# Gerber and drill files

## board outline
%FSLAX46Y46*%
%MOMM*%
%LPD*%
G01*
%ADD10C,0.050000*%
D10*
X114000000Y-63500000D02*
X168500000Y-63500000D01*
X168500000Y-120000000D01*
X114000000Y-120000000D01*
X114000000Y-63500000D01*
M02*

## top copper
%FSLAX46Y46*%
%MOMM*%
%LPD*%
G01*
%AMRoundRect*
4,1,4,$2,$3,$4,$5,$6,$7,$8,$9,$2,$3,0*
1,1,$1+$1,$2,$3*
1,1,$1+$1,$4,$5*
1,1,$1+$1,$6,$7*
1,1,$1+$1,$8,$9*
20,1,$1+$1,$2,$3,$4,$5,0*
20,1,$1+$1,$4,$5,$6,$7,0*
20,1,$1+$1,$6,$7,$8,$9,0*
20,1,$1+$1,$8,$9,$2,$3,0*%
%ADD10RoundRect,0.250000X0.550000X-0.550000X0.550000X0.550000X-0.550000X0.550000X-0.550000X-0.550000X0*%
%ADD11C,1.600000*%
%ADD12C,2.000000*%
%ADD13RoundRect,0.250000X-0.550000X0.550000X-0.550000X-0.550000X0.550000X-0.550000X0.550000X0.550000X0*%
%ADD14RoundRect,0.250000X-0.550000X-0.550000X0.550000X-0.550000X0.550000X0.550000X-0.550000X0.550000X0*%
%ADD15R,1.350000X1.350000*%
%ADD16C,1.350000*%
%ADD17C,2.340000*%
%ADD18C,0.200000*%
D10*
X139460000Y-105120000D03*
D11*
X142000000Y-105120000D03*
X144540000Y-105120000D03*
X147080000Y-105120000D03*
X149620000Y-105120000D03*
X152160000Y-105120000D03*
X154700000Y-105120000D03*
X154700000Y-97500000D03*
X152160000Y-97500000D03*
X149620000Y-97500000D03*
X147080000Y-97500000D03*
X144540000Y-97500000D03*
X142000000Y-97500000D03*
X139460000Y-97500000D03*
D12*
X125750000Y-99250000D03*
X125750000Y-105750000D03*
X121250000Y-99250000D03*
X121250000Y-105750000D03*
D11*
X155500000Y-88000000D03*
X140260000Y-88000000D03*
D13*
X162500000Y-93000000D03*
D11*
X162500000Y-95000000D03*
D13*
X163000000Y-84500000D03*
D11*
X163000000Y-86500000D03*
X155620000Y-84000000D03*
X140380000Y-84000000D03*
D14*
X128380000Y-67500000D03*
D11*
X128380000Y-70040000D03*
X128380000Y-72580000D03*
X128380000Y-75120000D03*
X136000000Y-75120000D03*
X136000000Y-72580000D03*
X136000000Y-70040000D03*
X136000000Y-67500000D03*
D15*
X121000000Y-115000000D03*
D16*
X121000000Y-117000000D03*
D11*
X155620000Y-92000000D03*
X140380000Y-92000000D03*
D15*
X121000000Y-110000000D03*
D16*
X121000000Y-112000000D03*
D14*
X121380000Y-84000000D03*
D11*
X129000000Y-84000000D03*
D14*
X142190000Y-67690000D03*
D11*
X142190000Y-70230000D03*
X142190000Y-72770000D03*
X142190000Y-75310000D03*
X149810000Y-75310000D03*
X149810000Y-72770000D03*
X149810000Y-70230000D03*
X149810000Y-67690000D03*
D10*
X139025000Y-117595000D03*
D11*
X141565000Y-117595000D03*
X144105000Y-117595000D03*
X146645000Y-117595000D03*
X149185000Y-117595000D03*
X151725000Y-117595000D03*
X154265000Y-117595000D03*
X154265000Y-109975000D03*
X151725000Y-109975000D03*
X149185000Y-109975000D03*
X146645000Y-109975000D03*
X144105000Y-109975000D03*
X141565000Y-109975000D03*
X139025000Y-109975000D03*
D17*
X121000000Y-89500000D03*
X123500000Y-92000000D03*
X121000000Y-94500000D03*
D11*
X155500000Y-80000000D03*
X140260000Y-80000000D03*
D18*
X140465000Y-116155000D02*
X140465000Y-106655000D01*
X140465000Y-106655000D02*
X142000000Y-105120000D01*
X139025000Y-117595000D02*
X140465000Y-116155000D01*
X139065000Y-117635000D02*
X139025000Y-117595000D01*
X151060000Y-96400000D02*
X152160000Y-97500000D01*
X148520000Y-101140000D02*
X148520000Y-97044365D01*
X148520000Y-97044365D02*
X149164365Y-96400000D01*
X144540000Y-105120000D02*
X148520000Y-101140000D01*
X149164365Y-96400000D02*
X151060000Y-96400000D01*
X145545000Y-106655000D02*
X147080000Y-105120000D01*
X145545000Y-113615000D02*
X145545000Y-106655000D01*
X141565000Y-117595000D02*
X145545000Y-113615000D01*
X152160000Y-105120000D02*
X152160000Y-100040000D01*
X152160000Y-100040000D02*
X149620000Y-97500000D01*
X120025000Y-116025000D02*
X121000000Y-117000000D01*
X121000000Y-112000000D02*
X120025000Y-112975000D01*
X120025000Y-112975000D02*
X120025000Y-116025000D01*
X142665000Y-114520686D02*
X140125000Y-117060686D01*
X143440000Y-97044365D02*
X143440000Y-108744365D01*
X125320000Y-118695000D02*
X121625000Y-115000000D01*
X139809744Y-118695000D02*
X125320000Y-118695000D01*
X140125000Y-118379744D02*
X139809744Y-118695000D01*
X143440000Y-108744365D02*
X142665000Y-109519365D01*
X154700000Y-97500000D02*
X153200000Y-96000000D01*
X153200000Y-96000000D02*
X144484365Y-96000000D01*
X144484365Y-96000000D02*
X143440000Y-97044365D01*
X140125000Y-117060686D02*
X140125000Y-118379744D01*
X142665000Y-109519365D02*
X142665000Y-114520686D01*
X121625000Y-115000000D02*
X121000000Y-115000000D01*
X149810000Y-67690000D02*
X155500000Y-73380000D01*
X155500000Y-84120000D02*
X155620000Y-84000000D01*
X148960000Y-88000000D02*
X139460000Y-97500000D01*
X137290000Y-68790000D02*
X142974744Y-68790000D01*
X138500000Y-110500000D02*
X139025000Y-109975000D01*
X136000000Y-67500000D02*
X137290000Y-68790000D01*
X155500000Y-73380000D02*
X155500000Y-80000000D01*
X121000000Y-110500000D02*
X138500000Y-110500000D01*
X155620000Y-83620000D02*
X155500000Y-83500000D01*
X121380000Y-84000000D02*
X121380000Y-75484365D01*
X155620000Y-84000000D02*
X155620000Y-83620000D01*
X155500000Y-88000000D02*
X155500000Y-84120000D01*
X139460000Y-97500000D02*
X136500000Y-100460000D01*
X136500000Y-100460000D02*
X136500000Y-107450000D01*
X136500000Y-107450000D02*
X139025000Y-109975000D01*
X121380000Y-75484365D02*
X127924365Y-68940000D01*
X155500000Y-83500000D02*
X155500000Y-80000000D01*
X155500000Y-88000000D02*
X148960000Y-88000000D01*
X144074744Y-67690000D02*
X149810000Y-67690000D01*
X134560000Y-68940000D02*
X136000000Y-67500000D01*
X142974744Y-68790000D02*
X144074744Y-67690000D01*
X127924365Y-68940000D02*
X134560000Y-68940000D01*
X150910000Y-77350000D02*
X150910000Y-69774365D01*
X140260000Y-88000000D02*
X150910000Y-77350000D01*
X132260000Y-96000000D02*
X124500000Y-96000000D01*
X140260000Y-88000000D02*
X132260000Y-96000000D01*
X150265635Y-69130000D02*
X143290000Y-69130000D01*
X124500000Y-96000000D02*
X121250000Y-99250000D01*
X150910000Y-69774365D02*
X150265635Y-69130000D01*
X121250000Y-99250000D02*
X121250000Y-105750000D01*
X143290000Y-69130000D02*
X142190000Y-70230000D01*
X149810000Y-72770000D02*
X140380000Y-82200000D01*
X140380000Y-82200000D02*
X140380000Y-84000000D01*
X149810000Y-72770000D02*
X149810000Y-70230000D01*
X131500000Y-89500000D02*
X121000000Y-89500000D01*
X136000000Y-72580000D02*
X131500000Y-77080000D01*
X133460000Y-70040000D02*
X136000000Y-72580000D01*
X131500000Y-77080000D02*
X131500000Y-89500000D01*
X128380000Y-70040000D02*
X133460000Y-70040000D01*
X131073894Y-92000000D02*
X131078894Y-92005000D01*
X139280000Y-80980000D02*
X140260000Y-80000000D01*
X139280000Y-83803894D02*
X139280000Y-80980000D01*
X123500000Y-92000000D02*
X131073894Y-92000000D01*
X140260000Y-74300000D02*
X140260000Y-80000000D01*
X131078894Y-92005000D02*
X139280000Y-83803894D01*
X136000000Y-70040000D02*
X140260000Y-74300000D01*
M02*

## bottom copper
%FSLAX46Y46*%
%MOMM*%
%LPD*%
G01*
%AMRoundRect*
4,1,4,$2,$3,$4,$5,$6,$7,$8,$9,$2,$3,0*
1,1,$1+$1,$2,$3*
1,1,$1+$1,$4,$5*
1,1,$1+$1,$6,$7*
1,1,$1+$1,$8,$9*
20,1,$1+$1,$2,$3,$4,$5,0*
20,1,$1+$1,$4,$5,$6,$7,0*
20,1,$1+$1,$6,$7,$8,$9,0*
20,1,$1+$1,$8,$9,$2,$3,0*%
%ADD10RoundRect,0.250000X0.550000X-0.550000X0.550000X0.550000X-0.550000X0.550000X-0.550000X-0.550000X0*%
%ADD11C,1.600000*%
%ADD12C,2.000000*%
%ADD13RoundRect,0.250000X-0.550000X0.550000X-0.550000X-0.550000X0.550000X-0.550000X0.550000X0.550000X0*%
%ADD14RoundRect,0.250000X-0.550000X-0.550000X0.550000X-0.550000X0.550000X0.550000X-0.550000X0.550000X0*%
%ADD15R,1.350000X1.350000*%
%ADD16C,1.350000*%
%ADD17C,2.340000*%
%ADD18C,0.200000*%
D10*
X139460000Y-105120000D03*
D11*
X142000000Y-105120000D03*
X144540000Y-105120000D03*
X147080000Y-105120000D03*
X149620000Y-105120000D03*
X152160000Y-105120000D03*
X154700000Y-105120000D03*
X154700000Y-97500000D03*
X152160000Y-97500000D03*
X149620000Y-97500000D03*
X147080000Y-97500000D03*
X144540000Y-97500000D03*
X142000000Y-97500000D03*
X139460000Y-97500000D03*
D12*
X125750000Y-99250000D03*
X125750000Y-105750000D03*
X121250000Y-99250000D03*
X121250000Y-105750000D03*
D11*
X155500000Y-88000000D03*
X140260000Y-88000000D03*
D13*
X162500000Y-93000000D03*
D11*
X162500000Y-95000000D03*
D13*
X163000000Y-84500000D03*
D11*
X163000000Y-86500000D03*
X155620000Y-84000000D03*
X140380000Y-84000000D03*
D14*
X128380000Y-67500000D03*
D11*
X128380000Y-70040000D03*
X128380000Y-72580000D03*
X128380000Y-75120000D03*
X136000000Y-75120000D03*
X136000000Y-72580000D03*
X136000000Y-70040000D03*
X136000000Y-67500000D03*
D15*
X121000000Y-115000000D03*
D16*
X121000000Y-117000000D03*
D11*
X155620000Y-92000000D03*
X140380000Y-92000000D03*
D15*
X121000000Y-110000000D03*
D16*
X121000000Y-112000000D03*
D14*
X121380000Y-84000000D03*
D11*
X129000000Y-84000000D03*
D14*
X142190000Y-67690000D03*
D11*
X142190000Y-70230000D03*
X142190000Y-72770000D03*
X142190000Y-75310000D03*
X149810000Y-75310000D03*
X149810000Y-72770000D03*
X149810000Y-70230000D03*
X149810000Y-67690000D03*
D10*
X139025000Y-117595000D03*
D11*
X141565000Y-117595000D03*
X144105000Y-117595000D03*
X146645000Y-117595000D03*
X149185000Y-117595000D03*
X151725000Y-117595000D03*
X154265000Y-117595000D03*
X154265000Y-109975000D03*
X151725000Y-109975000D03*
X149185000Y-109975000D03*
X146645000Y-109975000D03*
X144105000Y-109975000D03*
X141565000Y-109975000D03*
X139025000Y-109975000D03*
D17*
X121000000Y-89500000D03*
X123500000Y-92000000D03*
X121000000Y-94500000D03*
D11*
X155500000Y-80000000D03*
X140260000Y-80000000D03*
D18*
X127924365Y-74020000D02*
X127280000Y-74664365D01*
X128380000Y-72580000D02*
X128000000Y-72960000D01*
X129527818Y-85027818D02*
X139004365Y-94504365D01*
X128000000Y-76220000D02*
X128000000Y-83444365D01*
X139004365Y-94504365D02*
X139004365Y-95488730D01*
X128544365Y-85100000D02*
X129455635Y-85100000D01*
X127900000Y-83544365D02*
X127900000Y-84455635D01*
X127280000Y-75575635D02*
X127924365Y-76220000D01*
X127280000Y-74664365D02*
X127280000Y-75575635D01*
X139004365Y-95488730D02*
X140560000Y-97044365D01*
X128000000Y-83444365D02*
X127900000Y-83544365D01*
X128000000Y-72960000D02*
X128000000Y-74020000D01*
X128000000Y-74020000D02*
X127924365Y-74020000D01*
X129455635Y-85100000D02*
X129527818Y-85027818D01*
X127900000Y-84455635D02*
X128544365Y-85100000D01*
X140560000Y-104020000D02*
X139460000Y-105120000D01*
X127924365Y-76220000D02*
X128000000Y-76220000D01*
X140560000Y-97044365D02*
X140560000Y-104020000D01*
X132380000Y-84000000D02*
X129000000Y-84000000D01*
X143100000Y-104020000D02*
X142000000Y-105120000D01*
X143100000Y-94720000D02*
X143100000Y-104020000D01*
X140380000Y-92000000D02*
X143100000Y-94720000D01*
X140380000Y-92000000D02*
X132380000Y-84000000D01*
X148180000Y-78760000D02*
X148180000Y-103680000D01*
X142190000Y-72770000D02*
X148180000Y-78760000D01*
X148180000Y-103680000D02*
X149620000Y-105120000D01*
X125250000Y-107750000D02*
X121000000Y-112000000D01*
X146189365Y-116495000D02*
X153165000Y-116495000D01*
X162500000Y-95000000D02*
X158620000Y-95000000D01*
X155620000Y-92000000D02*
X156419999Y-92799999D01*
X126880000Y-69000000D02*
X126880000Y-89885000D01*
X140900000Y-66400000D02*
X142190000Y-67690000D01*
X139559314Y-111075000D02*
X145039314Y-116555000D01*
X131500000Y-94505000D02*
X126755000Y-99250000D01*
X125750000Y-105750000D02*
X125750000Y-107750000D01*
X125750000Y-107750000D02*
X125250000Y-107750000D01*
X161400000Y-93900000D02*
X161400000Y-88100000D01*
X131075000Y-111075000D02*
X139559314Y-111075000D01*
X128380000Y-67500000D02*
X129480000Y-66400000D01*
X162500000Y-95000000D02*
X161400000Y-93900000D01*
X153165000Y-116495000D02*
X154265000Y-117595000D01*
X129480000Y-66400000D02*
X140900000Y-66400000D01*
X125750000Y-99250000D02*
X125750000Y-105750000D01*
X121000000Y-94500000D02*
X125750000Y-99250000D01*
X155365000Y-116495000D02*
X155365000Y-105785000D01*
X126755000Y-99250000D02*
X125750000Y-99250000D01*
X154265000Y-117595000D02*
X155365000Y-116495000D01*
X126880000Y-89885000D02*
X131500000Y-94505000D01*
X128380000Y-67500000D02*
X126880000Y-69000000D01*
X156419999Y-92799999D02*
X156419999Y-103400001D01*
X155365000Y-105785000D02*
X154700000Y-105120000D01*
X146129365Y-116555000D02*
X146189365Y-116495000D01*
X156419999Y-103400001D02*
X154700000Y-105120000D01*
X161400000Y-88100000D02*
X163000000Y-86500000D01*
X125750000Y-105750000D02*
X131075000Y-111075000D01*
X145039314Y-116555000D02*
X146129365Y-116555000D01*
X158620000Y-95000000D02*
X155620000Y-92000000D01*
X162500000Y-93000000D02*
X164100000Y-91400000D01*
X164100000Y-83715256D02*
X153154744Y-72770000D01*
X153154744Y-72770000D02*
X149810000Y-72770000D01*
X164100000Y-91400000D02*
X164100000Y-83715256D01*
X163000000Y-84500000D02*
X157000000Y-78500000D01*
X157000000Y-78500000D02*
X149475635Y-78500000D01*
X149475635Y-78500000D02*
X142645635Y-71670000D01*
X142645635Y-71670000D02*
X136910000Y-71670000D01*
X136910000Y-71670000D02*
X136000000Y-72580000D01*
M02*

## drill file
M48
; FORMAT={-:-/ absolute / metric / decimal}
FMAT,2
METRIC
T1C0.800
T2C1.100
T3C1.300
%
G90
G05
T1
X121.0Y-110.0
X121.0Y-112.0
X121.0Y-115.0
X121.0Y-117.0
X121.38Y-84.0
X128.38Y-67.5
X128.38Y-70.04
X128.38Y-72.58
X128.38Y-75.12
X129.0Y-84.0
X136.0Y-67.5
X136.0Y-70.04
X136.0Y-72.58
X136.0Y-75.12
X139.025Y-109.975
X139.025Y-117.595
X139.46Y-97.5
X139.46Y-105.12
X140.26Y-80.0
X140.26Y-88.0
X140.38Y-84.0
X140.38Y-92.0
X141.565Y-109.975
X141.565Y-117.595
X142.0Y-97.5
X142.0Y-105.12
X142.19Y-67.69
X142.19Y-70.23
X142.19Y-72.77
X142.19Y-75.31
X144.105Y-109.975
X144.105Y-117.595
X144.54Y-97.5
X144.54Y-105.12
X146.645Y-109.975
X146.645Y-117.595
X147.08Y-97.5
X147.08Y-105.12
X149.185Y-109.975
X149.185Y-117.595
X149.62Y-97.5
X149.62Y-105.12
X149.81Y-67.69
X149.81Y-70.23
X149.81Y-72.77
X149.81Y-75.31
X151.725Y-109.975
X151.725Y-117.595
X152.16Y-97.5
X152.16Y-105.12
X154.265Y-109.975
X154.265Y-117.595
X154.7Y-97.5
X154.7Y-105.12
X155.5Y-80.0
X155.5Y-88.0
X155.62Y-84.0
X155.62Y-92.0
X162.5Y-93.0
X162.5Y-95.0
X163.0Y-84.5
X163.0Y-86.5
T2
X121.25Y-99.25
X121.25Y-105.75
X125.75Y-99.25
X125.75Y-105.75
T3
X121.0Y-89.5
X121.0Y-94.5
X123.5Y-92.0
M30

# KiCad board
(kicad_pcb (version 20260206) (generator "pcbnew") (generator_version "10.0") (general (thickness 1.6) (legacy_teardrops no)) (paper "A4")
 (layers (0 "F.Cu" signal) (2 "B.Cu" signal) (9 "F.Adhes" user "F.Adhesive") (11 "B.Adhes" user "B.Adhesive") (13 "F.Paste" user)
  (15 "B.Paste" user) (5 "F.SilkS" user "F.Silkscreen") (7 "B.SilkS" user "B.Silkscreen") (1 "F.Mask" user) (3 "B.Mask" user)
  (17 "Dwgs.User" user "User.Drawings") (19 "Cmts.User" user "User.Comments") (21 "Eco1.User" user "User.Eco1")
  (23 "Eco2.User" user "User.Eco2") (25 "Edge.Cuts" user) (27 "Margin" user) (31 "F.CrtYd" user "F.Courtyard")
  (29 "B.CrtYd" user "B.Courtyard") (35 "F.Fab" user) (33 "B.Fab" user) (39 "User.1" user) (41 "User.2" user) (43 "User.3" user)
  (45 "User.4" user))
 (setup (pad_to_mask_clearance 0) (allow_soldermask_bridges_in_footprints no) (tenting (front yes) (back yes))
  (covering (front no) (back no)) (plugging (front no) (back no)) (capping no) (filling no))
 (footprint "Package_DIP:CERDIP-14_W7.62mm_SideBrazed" (layer "F.Cu") (at 139.46 105.12 90)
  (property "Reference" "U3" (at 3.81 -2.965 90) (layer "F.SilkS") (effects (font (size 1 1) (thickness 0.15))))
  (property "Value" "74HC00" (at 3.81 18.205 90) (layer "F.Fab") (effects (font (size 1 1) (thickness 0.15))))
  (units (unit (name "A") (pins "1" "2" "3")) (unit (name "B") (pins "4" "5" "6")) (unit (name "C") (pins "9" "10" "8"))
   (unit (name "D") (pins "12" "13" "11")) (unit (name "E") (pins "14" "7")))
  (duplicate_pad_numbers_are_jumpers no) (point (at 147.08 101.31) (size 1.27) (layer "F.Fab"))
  (pad "1" thru_hole roundrect (at 0 0 90) (size 1.6 1.6) (drill 0.8) (layers "*.Cu" "*.Mask") (remove_unused_layers no)
   (roundrect_rratio 0.15625) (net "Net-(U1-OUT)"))
  (pad "2" thru_hole circle (at 0 2.54 90) (size 1.6 1.6) (drill 0.8) (layers "*.Cu" "*.Mask") (remove_unused_layers no)
   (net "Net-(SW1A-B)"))
  (pad "3" thru_hole circle (at 0 5.08 90) (size 1.6 1.6) (drill 0.8) (layers "*.Cu" "*.Mask") (remove_unused_layers no)
   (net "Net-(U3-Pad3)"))
  (pad "4" thru_hole circle (at 0 7.62 90) (size 1.6 1.6) (drill 0.8) (layers "*.Cu" "*.Mask") (remove_unused_layers no)
   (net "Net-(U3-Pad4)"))
  (pad "5" thru_hole circle (at 0 10.16 90) (size 1.6 1.6) (drill 0.8) (layers "*.Cu" "*.Mask") (remove_unused_layers no)
   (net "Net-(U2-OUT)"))
  (pad "6" thru_hole circle (at 0 12.7 90) (size 1.6 1.6) (drill 0.8) (layers "*.Cu" "*.Mask") (remove_unused_layers no)
   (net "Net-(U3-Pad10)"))
  (pad "7" thru_hole circle (at 0 15.24 90) (size 1.6 1.6) (drill 0.8) (layers "*.Cu" "*.Mask") (remove_unused_layers no) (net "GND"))
  (pad "8" thru_hole circle (at 7.62 15.24 90) (size 1.6 1.6) (drill 0.8) (layers "*.Cu" "*.Mask") (remove_unused_layers no)
   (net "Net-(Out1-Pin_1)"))
  (pad "9" thru_hole circle (at 7.62 12.7 90) (size 1.6 1.6) (drill 0.8) (layers "*.Cu" "*.Mask") (remove_unused_layers no)
   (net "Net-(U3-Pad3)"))
  (pad "10" thru_hole circle (at 7.62 10.16 90) (size 1.6 1.6) (drill 0.8) (layers "*.Cu" "*.Mask") (remove_unused_layers no)
   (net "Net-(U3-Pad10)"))
  (pad "11" thru_hole circle (at 7.62 7.62 90) (size 1.6 1.6) (drill 0.8) (layers "*.Cu" "*.Mask") (remove_unused_layers no))
  (pad "12" thru_hole circle (at 7.62 5.08 90) (size 1.6 1.6) (drill 0.8) (layers "*.Cu" "*.Mask") (remove_unused_layers no))
  (pad "13" thru_hole circle (at 7.62 2.54 90) (size 1.6 1.6) (drill 0.8) (layers "*.Cu" "*.Mask") (remove_unused_layers no))
  (pad "14" thru_hole circle (at 7.62 0 90) (size 1.6 1.6) (drill 0.8) (layers "*.Cu" "*.Mask") (remove_unused_layers no) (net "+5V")))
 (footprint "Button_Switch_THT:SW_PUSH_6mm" (layer "F.Cu") (at 125.75 99.25 -90)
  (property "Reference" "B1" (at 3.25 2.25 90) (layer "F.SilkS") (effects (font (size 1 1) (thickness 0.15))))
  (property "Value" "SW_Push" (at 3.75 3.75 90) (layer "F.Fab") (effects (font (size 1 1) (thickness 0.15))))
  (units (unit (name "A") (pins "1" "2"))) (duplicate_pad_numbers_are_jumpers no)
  (pad "1" thru_hole circle (at 0 0) (size 2 2) (drill 1.1) (layers "*.Cu" "*.Mask") (remove_unused_layers no) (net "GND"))
  (pad "1" thru_hole circle (at 6.5 0) (size 2 2) (drill 1.1) (layers "*.Cu" "*.Mask") (remove_unused_layers no) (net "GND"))
  (pad "2" thru_hole circle (at 0 4.5) (size 2 2) (drill 1.1) (layers "*.Cu" "*.Mask") (remove_unused_layers no) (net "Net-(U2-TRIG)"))
  (pad "2" thru_hole circle (at 6.5 4.5) (size 2 2) (drill 1.1) (layers "*.Cu" "*.Mask") (remove_unused_layers no) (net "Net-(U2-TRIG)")))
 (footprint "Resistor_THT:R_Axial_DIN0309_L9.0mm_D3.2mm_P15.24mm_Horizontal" (layer "F.Cu") (at 155.5 88 180)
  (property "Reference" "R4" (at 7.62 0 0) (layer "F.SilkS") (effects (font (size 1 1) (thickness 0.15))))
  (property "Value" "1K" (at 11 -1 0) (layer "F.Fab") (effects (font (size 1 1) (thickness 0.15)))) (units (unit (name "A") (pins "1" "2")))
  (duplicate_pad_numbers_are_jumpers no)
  (pad "1" thru_hole circle (at 0 0 180) (size 1.6 1.6) (drill 0.8) (layers "*.Cu" "*.Mask") (remove_unused_layers no) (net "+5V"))
  (pad "2" thru_hole circle (at 15.24 0 180) (size 1.6 1.6) (drill 0.8) (layers "*.Cu" "*.Mask") (remove_unused_layers no)
   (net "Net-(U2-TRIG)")))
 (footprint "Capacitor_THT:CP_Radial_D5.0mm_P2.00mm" (layer "F.Cu") (at 162.5 93 -90)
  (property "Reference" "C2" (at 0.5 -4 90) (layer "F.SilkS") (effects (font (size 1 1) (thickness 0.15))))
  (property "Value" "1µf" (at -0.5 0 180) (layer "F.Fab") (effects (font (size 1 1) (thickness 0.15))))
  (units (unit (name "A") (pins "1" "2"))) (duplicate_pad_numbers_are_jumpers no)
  (pad "1" thru_hole roundrect (at 0 0 270) (size 1.6 1.6) (drill 0.8) (layers "*.Cu" "*.Mask") (remove_unused_layers no)
   (roundrect_rratio 0.15625) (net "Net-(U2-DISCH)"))
  (pad "2" thru_hole circle (at 2 0 270) (size 1.6 1.6) (drill 0.8) (layers "*.Cu" "*.Mask") (remove_unused_layers no) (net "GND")))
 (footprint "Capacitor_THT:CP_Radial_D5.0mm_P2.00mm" (layer "F.Cu") (at 163 84.5 -90)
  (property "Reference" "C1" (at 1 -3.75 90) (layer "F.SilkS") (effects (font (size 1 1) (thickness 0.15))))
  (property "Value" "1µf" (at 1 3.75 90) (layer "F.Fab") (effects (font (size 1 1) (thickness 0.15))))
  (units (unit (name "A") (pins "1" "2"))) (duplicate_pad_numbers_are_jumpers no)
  (pad "1" thru_hole roundrect (at 0 0 270) (size 1.6 1.6) (drill 0.8) (layers "*.Cu" "*.Mask") (remove_unused_layers no)
   (roundrect_rratio 0.15625) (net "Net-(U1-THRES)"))
  (pad "2" thru_hole circle (at 2 0 270) (size 1.6 1.6) (drill 0.8) (layers "*.Cu" "*.Mask") (remove_unused_layers no) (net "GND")))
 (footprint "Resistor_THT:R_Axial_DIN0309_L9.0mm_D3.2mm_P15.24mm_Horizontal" (layer "F.Cu") (at 155.62 84 180)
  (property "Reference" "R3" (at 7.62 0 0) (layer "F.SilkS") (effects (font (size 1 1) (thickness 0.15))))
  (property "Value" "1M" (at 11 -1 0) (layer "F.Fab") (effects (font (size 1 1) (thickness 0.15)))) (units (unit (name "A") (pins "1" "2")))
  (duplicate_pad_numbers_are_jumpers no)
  (pad "1" thru_hole circle (at 0 0 180) (size 1.6 1.6) (drill 0.8) (layers "*.Cu" "*.Mask") (remove_unused_layers no) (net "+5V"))
  (pad "2" thru_hole circle (at 15.24 0 180) (size 1.6 1.6) (drill 0.8) (layers "*.Cu" "*.Mask") (remove_unused_layers no)
   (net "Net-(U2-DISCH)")))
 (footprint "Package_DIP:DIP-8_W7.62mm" (layer "F.Cu") (at 128.38 67.5)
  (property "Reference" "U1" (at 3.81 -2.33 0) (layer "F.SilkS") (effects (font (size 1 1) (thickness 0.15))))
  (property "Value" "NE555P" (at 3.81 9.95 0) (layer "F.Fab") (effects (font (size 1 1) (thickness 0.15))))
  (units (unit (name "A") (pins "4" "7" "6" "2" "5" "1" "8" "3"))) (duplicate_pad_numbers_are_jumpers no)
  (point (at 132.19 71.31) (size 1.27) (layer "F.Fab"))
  (pad "1" thru_hole roundrect (at 0 0) (size 1.6 1.6) (drill 0.8) (layers "*.Cu" "*.Mask") (remove_unused_layers no)
   (roundrect_rratio 0.15625) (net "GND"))
  (pad "2" thru_hole circle (at 0 2.54) (size 1.6 1.6) (drill 0.8) (layers "*.Cu" "*.Mask") (remove_unused_layers no) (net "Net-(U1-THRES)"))
  (pad "3" thru_hole circle (at 0 5.08) (size 1.6 1.6) (drill 0.8) (layers "*.Cu" "*.Mask") (remove_unused_layers no) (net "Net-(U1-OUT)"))
  (pad "4" thru_hole circle (at 0 7.62) (size 1.6 1.6) (drill 0.8) (layers "*.Cu" "*.Mask") (remove_unused_layers no)
   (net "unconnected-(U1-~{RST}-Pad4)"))
  (pad "5" thru_hole circle (at 7.62 7.62) (size 1.6 1.6) (drill 0.8) (layers "*.Cu" "*.Mask") (remove_unused_layers no)
   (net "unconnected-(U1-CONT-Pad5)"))
  (pad "6" thru_hole circle (at 7.62 5.08) (size 1.6 1.6) (drill 0.8) (layers "*.Cu" "*.Mask") (remove_unused_layers no)
   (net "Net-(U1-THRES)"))
  (pad "7" thru_hole circle (at 7.62 2.54) (size 1.6 1.6) (drill 0.8) (layers "*.Cu" "*.Mask") (remove_unused_layers no)
   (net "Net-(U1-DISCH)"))
  (pad "8" thru_hole circle (at 7.62 0) (size 1.6 1.6) (drill 0.8) (layers "*.Cu" "*.Mask") (remove_unused_layers no) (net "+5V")))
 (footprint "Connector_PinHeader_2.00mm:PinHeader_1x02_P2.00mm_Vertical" (layer "F.Cu") (at 121 115)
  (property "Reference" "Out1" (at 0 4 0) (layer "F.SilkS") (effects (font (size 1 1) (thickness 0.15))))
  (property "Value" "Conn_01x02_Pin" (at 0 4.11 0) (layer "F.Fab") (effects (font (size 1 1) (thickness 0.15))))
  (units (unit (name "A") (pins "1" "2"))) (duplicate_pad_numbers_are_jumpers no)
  (pad "1" thru_hole rect (at 0 0) (size 1.35 1.35) (drill 0.8) (layers "*.Cu" "*.Mask") (remove_unused_layers no) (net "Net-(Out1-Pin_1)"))
  (pad "2" thru_hole circle (at 0 2) (size 1.35 1.35) (drill 0.8) (layers "*.Cu" "*.Mask") (remove_unused_layers no) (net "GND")))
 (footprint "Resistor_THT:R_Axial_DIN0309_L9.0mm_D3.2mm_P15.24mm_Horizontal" (layer "F.Cu") (at 155.62 92 180)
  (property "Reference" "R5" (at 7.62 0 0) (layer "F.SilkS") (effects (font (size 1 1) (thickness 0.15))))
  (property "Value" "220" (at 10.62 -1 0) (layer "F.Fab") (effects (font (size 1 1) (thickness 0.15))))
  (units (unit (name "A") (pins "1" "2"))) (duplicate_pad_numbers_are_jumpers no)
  (pad "1" thru_hole circle (at 0 0 180) (size 1.6 1.6) (drill 0.8) (layers "*.Cu" "*.Mask") (remove_unused_layers no) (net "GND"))
  (pad "2" thru_hole circle (at 15.24 0 180) (size 1.6 1.6) (drill 0.8) (layers "*.Cu" "*.Mask") (remove_unused_layers no)
   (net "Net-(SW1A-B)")))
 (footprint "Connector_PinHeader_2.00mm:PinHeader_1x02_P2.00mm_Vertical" (layer "F.Cu") (at 121 110)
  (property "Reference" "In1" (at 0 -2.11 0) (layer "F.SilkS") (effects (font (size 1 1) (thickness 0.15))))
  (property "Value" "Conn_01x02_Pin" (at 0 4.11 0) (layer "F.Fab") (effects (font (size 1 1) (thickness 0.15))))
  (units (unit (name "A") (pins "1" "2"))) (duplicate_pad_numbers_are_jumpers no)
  (pad "1" thru_hole rect (at 0 0) (size 1.35 1.35) (drill 0.8) (layers "*.Cu" "*.Mask") (remove_unused_layers no) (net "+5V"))
  (pad "2" thru_hole circle (at 0 2) (size 1.35 1.35) (drill 0.8) (layers "*.Cu" "*.Mask") (remove_unused_layers no) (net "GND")))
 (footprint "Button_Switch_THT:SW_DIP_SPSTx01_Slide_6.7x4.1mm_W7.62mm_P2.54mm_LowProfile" (layer "F.Cu") (at 121.38 84)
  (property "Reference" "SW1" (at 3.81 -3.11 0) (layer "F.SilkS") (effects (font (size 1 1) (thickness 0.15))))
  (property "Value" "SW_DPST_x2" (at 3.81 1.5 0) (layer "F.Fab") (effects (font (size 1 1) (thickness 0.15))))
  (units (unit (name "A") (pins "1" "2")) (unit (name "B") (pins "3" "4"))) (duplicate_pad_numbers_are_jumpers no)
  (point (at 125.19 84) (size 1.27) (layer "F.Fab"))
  (pad "1" thru_hole roundrect (at 0 0) (size 1.6 1.6) (drill 0.8) (layers "*.Cu" "*.Mask") (remove_unused_layers no)
   (roundrect_rratio 0.15625) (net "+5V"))
  (pad "2" thru_hole circle (at 7.62 0) (size 1.6 1.6) (drill 0.8) (layers "*.Cu" "*.Mask") (remove_unused_layers no) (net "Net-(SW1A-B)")))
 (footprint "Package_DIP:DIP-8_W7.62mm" (layer "F.Cu") (at 142.19 67.69)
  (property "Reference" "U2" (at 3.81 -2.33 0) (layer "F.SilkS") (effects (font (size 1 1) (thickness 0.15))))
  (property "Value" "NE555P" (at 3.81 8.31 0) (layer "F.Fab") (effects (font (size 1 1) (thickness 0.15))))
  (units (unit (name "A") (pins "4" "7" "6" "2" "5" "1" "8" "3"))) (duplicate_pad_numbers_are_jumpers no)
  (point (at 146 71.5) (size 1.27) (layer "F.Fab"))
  (pad "1" thru_hole roundrect (at 0 0) (size 1.6 1.6) (drill 0.8) (layers "*.Cu" "*.Mask") (remove_unused_layers no)
   (roundrect_rratio 0.15625) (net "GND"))
  (pad "2" thru_hole circle (at 0 2.54) (size 1.6 1.6) (drill 0.8) (layers "*.Cu" "*.Mask") (remove_unused_layers no) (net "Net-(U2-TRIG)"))
  (pad "3" thru_hole circle (at 0 5.08) (size 1.6 1.6) (drill 0.8) (layers "*.Cu" "*.Mask") (remove_unused_layers no) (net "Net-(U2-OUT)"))
  (pad "4" thru_hole circle (at 0 7.62) (size 1.6 1.6) (drill 0.8) (layers "*.Cu" "*.Mask") (remove_unused_layers no)
   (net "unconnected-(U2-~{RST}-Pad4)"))
  (pad "5" thru_hole circle (at 7.62 7.62) (size 1.6 1.6) (drill 0.8) (layers "*.Cu" "*.Mask") (remove_unused_layers no)
   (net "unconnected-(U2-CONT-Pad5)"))
  (pad "6" thru_hole circle (at 7.62 5.08) (size 1.6 1.6) (drill 0.8) (layers "*.Cu" "*.Mask") (remove_unused_layers no)
   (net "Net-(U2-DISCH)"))
  (pad "7" thru_hole circle (at 7.62 2.54) (size 1.6 1.6) (drill 0.8) (layers "*.Cu" "*.Mask") (remove_unused_layers no)
   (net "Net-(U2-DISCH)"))
  (pad "8" thru_hole circle (at 7.62 0) (size 1.6 1.6) (drill 0.8) (layers "*.Cu" "*.Mask") (remove_unused_layers no) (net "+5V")))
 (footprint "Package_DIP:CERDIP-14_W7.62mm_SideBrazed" (layer "F.Cu") (at 139.025 117.595 90)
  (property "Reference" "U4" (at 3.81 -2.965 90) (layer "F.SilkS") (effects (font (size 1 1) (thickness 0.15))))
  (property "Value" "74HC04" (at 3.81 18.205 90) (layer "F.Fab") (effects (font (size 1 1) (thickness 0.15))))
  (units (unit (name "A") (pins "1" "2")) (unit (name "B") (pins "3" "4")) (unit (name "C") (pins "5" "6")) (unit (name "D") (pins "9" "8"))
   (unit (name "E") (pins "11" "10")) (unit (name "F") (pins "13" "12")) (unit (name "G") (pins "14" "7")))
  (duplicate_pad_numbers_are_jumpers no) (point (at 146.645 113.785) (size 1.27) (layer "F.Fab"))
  (pad "1" thru_hole roundrect (at 0 0 90) (size 1.6 1.6) (drill 0.8) (layers "*.Cu" "*.Mask") (remove_unused_layers no)
   (roundrect_rratio 0.15625) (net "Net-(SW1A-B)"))
  (pad "2" thru_hole circle (at 0 2.54 90) (size 1.6 1.6) (drill 0.8) (layers "*.Cu" "*.Mask") (remove_unused_layers no)
   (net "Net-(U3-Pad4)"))
  (pad "3" thru_hole circle (at 0 5.08 90) (size 1.6 1.6) (drill 0.8) (layers "*.Cu" "*.Mask") (remove_unused_layers no))
  (pad "4" thru_hole circle (at 0 7.62 90) (size 1.6 1.6) (drill 0.8) (layers "*.Cu" "*.Mask") (remove_unused_layers no))
  (pad "5" thru_hole circle (at 0 10.16 90) (size 1.6 1.6) (drill 0.8) (layers "*.Cu" "*.Mask") (remove_unused_layers no))
  (pad "6" thru_hole circle (at 0 12.7 90) (size 1.6 1.6) (drill 0.8) (layers "*.Cu" "*.Mask") (remove_unused_layers no))
  (pad "7" thru_hole circle (at 0 15.24 90) (size 1.6 1.6) (drill 0.8) (layers "*.Cu" "*.Mask") (remove_unused_layers no) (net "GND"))
  (pad "8" thru_hole circle (at 7.62 15.24 90) (size 1.6 1.6) (drill 0.8) (layers "*.Cu" "*.Mask") (remove_unused_layers no))
  (pad "9" thru_hole circle (at 7.62 12.7 90) (size 1.6 1.6) (drill 0.8) (layers "*.Cu" "*.Mask") (remove_unused_layers no))
  (pad "10" thru_hole circle (at 7.62 10.16 90) (size 1.6 1.6) (drill 0.8) (layers "*.Cu" "*.Mask") (remove_unused_layers no))
  (pad "11" thru_hole circle (at 7.62 7.62 90) (size 1.6 1.6) (drill 0.8) (layers "*.Cu" "*.Mask") (remove_unused_layers no))
  (pad "12" thru_hole circle (at 7.62 5.08 90) (size 1.6 1.6) (drill 0.8) (layers "*.Cu" "*.Mask") (remove_unused_layers no))
  (pad "13" thru_hole circle (at 7.62 2.54 90) (size 1.6 1.6) (drill 0.8) (layers "*.Cu" "*.Mask") (remove_unused_layers no))
  (pad "14" thru_hole circle (at 7.62 0 90) (size 1.6 1.6) (drill 0.8) (layers "*.Cu" "*.Mask") (remove_unused_layers no) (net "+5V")))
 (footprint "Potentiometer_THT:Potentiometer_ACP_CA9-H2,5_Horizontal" (layer "F.Cu") (at 121 89.5)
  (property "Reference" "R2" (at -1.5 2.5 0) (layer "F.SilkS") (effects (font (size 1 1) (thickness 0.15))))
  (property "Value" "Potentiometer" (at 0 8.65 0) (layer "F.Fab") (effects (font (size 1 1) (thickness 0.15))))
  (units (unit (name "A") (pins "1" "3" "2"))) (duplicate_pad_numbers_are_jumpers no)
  (pad "1" thru_hole circle (at 0 0) (size 2.34 2.34) (drill 1.3) (layers "*.Cu" "*.Mask") (remove_unused_layers no) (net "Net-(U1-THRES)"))
  (pad "2" thru_hole circle (at 2.5 2.5) (size 2.34 2.34) (drill 1.3) (layers "*.Cu" "*.Mask") (remove_unused_layers no)
   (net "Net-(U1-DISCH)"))
  (pad "3" thru_hole circle (at 0 5) (size 2.34 2.34) (drill 1.3) (layers "*.Cu" "*.Mask") (remove_unused_layers no) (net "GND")))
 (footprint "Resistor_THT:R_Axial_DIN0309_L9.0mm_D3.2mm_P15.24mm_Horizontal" (layer "F.Cu") (at 155.5 80 180)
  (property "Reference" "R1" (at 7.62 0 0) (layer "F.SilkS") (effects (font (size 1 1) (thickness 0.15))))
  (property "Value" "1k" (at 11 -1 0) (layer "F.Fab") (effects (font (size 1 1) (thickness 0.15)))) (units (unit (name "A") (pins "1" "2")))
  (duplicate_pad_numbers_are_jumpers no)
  (pad "1" thru_hole circle (at 0 0 180) (size 1.6 1.6) (drill 0.8) (layers "*.Cu" "*.Mask") (remove_unused_layers no) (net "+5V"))
  (pad "2" thru_hole circle (at 15.24 0 180) (size 1.6 1.6) (drill 0.8) (layers "*.Cu" "*.Mask") (remove_unused_layers no)
   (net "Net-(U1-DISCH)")))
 (gr_rect (start 114 63.5) (end 168.5 120) (stroke (width 0.05) (type default)) (fill no) (layer "Edge.Cuts"))
 (segment (start 127.924365 74.02) (end 127.28 74.664365) (width 0.2) (layer "B.Cu") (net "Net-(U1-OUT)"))
 (segment (start 128.38 72.58) (end 128 72.96) (width 0.2) (layer "B.Cu") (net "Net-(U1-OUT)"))
 (segment (start 129.527818 85.027818) (end 139.004365 94.504365) (width 0.2) (layer "B.Cu") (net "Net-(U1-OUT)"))
 (segment (start 128 76.22) (end 128 83.444365) (width 0.2) (layer "B.Cu") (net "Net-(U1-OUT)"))
 (segment (start 139.004365 94.504365) (end 139.004365 95.48873) (width 0.2) (layer "B.Cu") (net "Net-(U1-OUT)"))
 (segment (start 128.544365 85.1) (end 129.455635 85.1) (width 0.2) (layer "B.Cu") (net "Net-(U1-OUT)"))
 (segment (start 127.9 83.544365) (end 127.9 84.455635) (width 0.2) (layer "B.Cu") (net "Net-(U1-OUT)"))
 (segment (start 127.28 75.575635) (end 127.924365 76.22) (width 0.2) (layer "B.Cu") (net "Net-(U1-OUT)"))
 (segment (start 127.28 74.664365) (end 127.28 75.575635) (width 0.2) (layer "B.Cu") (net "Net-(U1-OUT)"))
 (segment (start 139.004365 95.48873) (end 140.56 97.044365) (width 0.2) (layer "B.Cu") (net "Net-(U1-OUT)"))
 (segment (start 128 83.444365) (end 127.9 83.544365) (width 0.2) (layer "B.Cu") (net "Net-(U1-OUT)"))
 (segment (start 128 72.96) (end 128 74.02) (width 0.2) (layer "B.Cu") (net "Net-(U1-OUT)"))
 (segment (start 128 74.02) (end 127.924365 74.02) (width 0.2) (layer "B.Cu") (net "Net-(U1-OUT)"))
 (segment (start 129.455635 85.1) (end 129.527818 85.027818) (width 0.2) (layer "B.Cu") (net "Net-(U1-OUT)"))
 (segment (start 127.9 84.455635) (end 128.544365 85.1) (width 0.2) (layer "B.Cu") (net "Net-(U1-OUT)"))
 (segment (start 140.56 104.02) (end 139.46 105.12) (width 0.2) (layer "B.Cu") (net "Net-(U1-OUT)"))
 (segment (start 127.924365 76.22) (end 128 76.22) (width 0.2) (layer "B.Cu") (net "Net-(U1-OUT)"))
 (segment (start 140.56 97.044365) (end 140.56 104.02) (width 0.2) (layer "B.Cu") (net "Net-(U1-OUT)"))
 (segment (start 140.465 116.155) (end 140.465 106.655) (width 0.2) (layer "F.Cu") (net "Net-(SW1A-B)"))
 (segment (start 140.465 106.655) (end 142 105.12) (width 0.2) (layer "F.Cu") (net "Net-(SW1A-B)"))
 (segment (start 139.025 117.595) (end 140.465 116.155) (width 0.2) (layer "F.Cu") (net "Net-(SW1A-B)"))
 (segment (start 139.065 117.635) (end 139.025 117.595) (width 0.2) (layer "F.Cu") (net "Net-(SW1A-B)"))
 (segment (start 132.38 84) (end 129 84) (width 0.2) (layer "B.Cu") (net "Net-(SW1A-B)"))
 (segment (start 143.1 104.02) (end 142 105.12) (width 0.2) (layer "B.Cu") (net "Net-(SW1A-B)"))
 (segment (start 143.1 94.72) (end 143.1 104.02) (width 0.2) (layer "B.Cu") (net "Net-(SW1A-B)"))
 (segment (start 140.38 92) (end 143.1 94.72) (width 0.2) (layer "B.Cu") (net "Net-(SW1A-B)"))
 (segment (start 140.38 92) (end 132.38 84) (width 0.2) (layer "B.Cu") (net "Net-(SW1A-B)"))
 (segment (start 151.06 96.4) (end 152.16 97.5) (width 0.2) (layer "F.Cu") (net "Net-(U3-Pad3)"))
 (segment (start 148.52 101.14) (end 148.52 97.044365) (width 0.2) (layer "F.Cu") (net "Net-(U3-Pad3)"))
 (segment (start 148.52 97.044365) (end 149.164365 96.4) (width 0.2) (layer "F.Cu") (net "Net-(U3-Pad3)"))
 (segment (start 144.54 105.12) (end 148.52 101.14) (width 0.2) (layer "F.Cu") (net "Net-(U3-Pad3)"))
 (segment (start 149.164365 96.4) (end 151.06 96.4) (width 0.2) (layer "F.Cu") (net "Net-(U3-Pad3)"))
 (segment (start 145.545 106.655) (end 147.08 105.12) (width 0.2) (layer "F.Cu") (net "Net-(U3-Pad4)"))
 (segment (start 145.545 113.615) (end 145.545 106.655) (width 0.2) (layer "F.Cu") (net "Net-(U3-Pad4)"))
 (segment (start 141.565 117.595) (end 145.545 113.615) (width 0.2) (layer "F.Cu") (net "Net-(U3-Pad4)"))
 (segment (start 148.18 78.76) (end 148.18 103.68) (width 0.2) (layer "B.Cu") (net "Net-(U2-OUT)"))
 (segment (start 142.19 72.77) (end 148.18 78.76) (width 0.2) (layer "B.Cu") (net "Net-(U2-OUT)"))
 (segment (start 148.18 103.68) (end 149.62 105.12) (width 0.2) (layer "B.Cu") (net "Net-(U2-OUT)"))
 (segment (start 152.16 105.12) (end 152.16 100.04) (width 0.2) (layer "F.Cu") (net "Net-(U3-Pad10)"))
 (segment (start 152.16 100.04) (end 149.62 97.5) (width 0.2) (layer "F.Cu") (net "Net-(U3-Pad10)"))
 (segment (start 120.025 116.025) (end 121 117) (width 0.2) (layer "F.Cu") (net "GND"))
 (segment (start 121 112) (end 120.025 112.975) (width 0.2) (layer "F.Cu") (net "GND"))
 (segment (start 120.025 112.975) (end 120.025 116.025) (width 0.2) (layer "F.Cu") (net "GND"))
 (segment (start 125.25 107.75) (end 121 112) (width 0.2) (layer "B.Cu") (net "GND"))
 (segment (start 146.189365 116.495) (end 153.165 116.495) (width 0.2) (layer "B.Cu") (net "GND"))
 (segment (start 162.5 95) (end 158.62 95) (width 0.2) (layer "B.Cu") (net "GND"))
 (segment (start 155.62 92) (end 156.419999 92.799999) (width 0.2) (layer "B.Cu") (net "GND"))
 (segment (start 126.88 69) (end 126.88 89.885) (width 0.2) (layer "B.Cu") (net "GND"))
 (segment (start 140.9 66.4) (end 142.19 67.69) (width 0.2) (layer "B.Cu") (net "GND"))
 (segment (start 139.559314 111.075) (end 145.039314 116.555) (width 0.2) (layer "B.Cu") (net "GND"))
 (segment (start 131.5 94.505) (end 126.755 99.25) (width 0.2) (layer "B.Cu") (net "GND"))
 (segment (start 125.75 105.75) (end 125.75 107.75) (width 0.2) (layer "B.Cu") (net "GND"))
 (segment (start 125.75 107.75) (end 125.25 107.75) (width 0.2) (layer "B.Cu") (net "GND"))
 (segment (start 161.4 93.9) (end 161.4 88.1) (width 0.2) (layer "B.Cu") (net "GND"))
 (segment (start 131.075 111.075) (end 139.559314 111.075) (width 0.2) (layer "B.Cu") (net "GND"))
 (segment (start 128.38 67.5) (end 129.48 66.4) (width 0.2) (layer "B.Cu") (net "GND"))
 (segment (start 162.5 95) (end 161.4 93.9) (width 0.2) (layer "B.Cu") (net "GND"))
 (segment (start 153.165 116.495) (end 154.265 117.595) (width 0.2) (layer "B.Cu") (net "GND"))
 (segment (start 129.48 66.4) (end 140.9 66.4) (width 0.2) (layer "B.Cu") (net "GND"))
 (segment (start 125.75 99.25) (end 125.75 105.75) (width 0.2) (layer "B.Cu") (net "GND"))
 (segment (start 121 94.5) (end 125.75 99.25) (width 0.2) (layer "B.Cu") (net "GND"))
 (segment (start 155.365 116.495) (end 155.365 105.785) (width 0.2) (layer "B.Cu") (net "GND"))
 (segment (start 126.755 99.25) (end 125.75 99.25) (width 0.2) (layer "B.Cu") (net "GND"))
 (segment (start 154.265 117.595) (end 155.365 116.495) (width 0.2) (layer "B.Cu") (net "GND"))
 (segment (start 126.88 89.885) (end 131.5 94.505) (width 0.2) (layer "B.Cu") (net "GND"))
 (segment (start 128.38 67.5) (end 126.88 69) (width 0.2) (layer "B.Cu") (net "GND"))
 (segment (start 156.419999 92.799999) (end 156.419999 103.400001) (width 0.2) (layer "B.Cu") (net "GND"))
 (segment (start 155.365 105.785) (end 154.7 105.12) (width 0.2) (layer "B.Cu") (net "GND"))
 (segment (start 146.129365 116.555) (end 146.189365 116.495) (width 0.2) (layer "B.Cu") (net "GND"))
 (segment (start 156.419999 103.400001) (end 154.7 105.12) (width 0.2) (layer "B.Cu") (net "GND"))
 (segment (start 161.4 88.1) (end 163 86.5) (width 0.2) (layer "B.Cu") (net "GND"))
 (segment (start 125.75 105.75) (end 131.075 111.075) (width 0.2) (layer "B.Cu") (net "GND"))
 (segment (start 145.039314 116.555) (end 146.129365 116.555) (width 0.2) (layer "B.Cu") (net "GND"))
 (segment (start 158.62 95) (end 155.62 92) (width 0.2) (layer "B.Cu") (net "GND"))
 (segment (start 142.665 114.520686) (end 140.125 117.060686) (width 0.2) (layer "F.Cu") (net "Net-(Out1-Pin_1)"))
 (segment (start 143.44 97.044365) (end 143.44 108.744365) (width 0.2) (layer "F.Cu") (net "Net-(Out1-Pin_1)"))
 (segment (start 125.32 118.695) (end 121.625 115) (width 0.2) (layer "F.Cu") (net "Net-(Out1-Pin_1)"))
 (segment (start 139.809744 118.695) (end 125.32 118.695) (width 0.2) (layer "F.Cu") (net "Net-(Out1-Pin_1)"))
 (segment (start 140.125 118.379744) (end 139.809744 118.695) (width 0.2) (layer "F.Cu") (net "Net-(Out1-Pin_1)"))
 (segment (start 143.44 108.744365) (end 142.665 109.519365) (width 0.2) (layer "F.Cu") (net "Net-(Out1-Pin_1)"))
 (segment (start 154.7 97.5) (end 153.2 96) (width 0.2) (layer "F.Cu") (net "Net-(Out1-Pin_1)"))
 (segment (start 153.2 96) (end 144.484365 96) (width 0.2) (layer "F.Cu") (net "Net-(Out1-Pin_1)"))
 (segment (start 144.484365 96) (end 143.44 97.044365) (width 0.2) (layer "F.Cu") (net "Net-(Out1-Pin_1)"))
 (segment (start 140.125 117.060686) (end 140.125 118.379744) (width 0.2) (layer "F.Cu") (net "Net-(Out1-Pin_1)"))
 (segment (start 142.665 109.519365) (end 142.665 114.520686) (width 0.2) (layer "F.Cu") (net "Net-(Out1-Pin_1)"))
 (segment (start 121.625 115) (end 121 115) (width 0.2) (layer "F.Cu") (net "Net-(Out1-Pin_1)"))
 (segment (start 149.81 67.69) (end 155.5 73.38) (width 0.2) (layer "F.Cu") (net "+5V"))
 (segment (start 155.5 84.12) (end 155.62 84) (width 0.2) (layer "F.Cu") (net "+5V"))
 (segment (start 148.96 88) (end 139.46 97.5) (width 0.2) (layer "F.Cu") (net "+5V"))
 (segment (start 137.29 68.79) (end 142.974744 68.79) (width 0.2) (layer "F.Cu") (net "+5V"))
 (segment (start 138.5 110.5) (end 139.025 109.975) (width 0.2) (layer "F.Cu") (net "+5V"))
 (segment (start 136 67.5) (end 137.29 68.79) (width 0.2) (layer "F.Cu") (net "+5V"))
 (segment (start 155.5 73.38) (end 155.5 80) (width 0.2) (layer "F.Cu") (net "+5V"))
 (segment (start 121 110.5) (end 138.5 110.5) (width 0.2) (layer "F.Cu") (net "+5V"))
 (segment (start 155.62 83.62) (end 155.5 83.5) (width 0.2) (layer "F.Cu") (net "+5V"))
 (segment (start 121.38 84) (end 121.38 75.484365) (width 0.2) (layer "F.Cu") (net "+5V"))
 (segment (start 155.62 84) (end 155.62 83.62) (width 0.2) (layer "F.Cu") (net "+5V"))
 (segment (start 155.5 88) (end 155.5 84.12) (width 0.2) (layer "F.Cu") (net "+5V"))
 (segment (start 139.46 97.5) (end 136.5 100.46) (width 0.2) (layer "F.Cu") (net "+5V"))
 (segment (start 136.5 100.46) (end 136.5 107.45) (width 0.2) (layer "F.Cu") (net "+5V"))
 (segment (start 136.5 107.45) (end 139.025 109.975) (width 0.2) (layer "F.Cu") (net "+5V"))
 (segment (start 121.38 75.484365) (end 127.924365 68.94) (width 0.2) (layer "F.Cu") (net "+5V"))
 (segment (start 155.5 83.5) (end 155.5 80) (width 0.2) (layer "F.Cu") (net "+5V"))
 (segment (start 155.5 88) (end 148.96 88) (width 0.2) (layer "F.Cu") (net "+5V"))
 (segment (start 144.074744 67.69) (end 149.81 67.69) (width 0.2) (layer "F.Cu") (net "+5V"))
 (segment (start 134.56 68.94) (end 136 67.5) (width 0.2) (layer "F.Cu") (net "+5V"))
 (segment (start 142.974744 68.79) (end 144.074744 67.69) (width 0.2) (layer "F.Cu") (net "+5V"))
 (segment (start 127.924365 68.94) (end 134.56 68.94) (width 0.2) (layer "F.Cu") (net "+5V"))
 (segment (start 150.91 77.35) (end 150.91 69.774365) (width 0.2) (layer "F.Cu") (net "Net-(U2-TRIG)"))
 (segment (start 140.26 88) (end 150.91 77.35) (width 0.2) (layer "F.Cu") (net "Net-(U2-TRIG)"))
 (segment (start 132.26 96) (end 124.5 96) (width 0.2) (layer "F.Cu") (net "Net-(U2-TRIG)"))
 (segment (start 140.26 88) (end 132.26 96) (width 0.2) (layer "F.Cu") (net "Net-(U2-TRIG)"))
 (segment (start 150.265635 69.13) (end 143.29 69.13) (width 0.2) (layer "F.Cu") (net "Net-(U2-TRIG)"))
 (segment (start 124.5 96) (end 121.25 99.25) (width 0.2) (layer "F.Cu") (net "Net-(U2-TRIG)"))
 (segment (start 150.91 69.774365) (end 150.265635 69.13) (width 0.2) (layer "F.Cu") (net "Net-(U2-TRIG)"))
 (segment (start 121.25 99.25) (end 121.25 105.75) (width 0.2) (layer "F.Cu") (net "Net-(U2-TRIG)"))
 (segment (start 143.29 69.13) (end 142.19 70.23) (width 0.2) (layer "F.Cu") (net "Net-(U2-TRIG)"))
 (segment (start 149.81 72.77) (end 140.38 82.2) (width 0.2) (layer "F.Cu") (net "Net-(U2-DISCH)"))
 (segment (start 140.38 82.2) (end 140.38 84) (width 0.2) (layer "F.Cu") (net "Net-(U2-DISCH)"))
 (segment (start 149.81 72.77) (end 149.81 70.23) (width 0.2) (layer "F.Cu") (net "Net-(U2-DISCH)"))
 (segment (start 162.5 93) (end 164.1 91.4) (width 0.2) (layer "B.Cu") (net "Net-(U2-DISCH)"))
 (segment (start 164.1 83.715256) (end 153.154744 72.77) (width 0.2) (layer "B.Cu") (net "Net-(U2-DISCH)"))
 (segment (start 153.154744 72.77) (end 149.81 72.77) (width 0.2) (layer "B.Cu") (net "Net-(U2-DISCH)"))
 (segment (start 164.1 91.4) (end 164.1 83.715256) (width 0.2) (layer "B.Cu") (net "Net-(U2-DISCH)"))
 (segment (start 131.5 89.5) (end 121 89.5) (width 0.2) (layer "F.Cu") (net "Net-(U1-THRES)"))
 (segment (start 136 72.58) (end 131.5 77.08) (width 0.2) (layer "F.Cu") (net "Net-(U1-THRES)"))
 (segment (start 133.46 70.04) (end 136 72.58) (width 0.2) (layer "F.Cu") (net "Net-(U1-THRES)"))
 (segment (start 131.5 77.08) (end 131.5 89.5) (width 0.2) (layer "F.Cu") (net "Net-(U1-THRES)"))
 (segment (start 128.38 70.04) (end 133.46 70.04) (width 0.2) (layer "F.Cu") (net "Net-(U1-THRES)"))
 (segment (start 163 84.5) (end 157 78.5) (width 0.2) (layer "B.Cu") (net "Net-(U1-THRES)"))
 (segment (start 157 78.5) (end 149.475635 78.5) (width 0.2) (layer "B.Cu") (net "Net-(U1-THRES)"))
 (segment (start 149.475635 78.5) (end 142.645635 71.67) (width 0.2) (layer "B.Cu") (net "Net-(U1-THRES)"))
 (segment (start 142.645635 71.67) (end 136.91 71.67) (width 0.2) (layer "B.Cu") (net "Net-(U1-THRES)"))
 (segment (start 136.91 71.67) (end 136 72.58) (width 0.2) (layer "B.Cu") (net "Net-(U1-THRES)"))
 (segment (start 131.073894 92) (end 131.078894 92.005) (width 0.2) (layer "F.Cu") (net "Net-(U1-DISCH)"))
 (segment (start 139.28 80.98) (end 140.26 80) (width 0.2) (layer "F.Cu") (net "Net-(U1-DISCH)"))
 (segment (start 139.28 83.803894) (end 139.28 80.98) (width 0.2) (layer "F.Cu") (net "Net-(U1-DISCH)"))
 (segment (start 123.5 92) (end 131.073894 92) (width 0.2) (layer "F.Cu") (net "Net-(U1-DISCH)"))
 (segment (start 140.26 74.3) (end 140.26 80) (width 0.2) (layer "F.Cu") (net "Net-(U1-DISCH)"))
 (segment (start 131.078894 92.005) (end 139.28 83.803894) (width 0.2) (layer "F.Cu") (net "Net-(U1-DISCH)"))
 (segment (start 136 70.04) (end 140.26 74.3) (width 0.2) (layer "F.Cu") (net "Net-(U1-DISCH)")))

